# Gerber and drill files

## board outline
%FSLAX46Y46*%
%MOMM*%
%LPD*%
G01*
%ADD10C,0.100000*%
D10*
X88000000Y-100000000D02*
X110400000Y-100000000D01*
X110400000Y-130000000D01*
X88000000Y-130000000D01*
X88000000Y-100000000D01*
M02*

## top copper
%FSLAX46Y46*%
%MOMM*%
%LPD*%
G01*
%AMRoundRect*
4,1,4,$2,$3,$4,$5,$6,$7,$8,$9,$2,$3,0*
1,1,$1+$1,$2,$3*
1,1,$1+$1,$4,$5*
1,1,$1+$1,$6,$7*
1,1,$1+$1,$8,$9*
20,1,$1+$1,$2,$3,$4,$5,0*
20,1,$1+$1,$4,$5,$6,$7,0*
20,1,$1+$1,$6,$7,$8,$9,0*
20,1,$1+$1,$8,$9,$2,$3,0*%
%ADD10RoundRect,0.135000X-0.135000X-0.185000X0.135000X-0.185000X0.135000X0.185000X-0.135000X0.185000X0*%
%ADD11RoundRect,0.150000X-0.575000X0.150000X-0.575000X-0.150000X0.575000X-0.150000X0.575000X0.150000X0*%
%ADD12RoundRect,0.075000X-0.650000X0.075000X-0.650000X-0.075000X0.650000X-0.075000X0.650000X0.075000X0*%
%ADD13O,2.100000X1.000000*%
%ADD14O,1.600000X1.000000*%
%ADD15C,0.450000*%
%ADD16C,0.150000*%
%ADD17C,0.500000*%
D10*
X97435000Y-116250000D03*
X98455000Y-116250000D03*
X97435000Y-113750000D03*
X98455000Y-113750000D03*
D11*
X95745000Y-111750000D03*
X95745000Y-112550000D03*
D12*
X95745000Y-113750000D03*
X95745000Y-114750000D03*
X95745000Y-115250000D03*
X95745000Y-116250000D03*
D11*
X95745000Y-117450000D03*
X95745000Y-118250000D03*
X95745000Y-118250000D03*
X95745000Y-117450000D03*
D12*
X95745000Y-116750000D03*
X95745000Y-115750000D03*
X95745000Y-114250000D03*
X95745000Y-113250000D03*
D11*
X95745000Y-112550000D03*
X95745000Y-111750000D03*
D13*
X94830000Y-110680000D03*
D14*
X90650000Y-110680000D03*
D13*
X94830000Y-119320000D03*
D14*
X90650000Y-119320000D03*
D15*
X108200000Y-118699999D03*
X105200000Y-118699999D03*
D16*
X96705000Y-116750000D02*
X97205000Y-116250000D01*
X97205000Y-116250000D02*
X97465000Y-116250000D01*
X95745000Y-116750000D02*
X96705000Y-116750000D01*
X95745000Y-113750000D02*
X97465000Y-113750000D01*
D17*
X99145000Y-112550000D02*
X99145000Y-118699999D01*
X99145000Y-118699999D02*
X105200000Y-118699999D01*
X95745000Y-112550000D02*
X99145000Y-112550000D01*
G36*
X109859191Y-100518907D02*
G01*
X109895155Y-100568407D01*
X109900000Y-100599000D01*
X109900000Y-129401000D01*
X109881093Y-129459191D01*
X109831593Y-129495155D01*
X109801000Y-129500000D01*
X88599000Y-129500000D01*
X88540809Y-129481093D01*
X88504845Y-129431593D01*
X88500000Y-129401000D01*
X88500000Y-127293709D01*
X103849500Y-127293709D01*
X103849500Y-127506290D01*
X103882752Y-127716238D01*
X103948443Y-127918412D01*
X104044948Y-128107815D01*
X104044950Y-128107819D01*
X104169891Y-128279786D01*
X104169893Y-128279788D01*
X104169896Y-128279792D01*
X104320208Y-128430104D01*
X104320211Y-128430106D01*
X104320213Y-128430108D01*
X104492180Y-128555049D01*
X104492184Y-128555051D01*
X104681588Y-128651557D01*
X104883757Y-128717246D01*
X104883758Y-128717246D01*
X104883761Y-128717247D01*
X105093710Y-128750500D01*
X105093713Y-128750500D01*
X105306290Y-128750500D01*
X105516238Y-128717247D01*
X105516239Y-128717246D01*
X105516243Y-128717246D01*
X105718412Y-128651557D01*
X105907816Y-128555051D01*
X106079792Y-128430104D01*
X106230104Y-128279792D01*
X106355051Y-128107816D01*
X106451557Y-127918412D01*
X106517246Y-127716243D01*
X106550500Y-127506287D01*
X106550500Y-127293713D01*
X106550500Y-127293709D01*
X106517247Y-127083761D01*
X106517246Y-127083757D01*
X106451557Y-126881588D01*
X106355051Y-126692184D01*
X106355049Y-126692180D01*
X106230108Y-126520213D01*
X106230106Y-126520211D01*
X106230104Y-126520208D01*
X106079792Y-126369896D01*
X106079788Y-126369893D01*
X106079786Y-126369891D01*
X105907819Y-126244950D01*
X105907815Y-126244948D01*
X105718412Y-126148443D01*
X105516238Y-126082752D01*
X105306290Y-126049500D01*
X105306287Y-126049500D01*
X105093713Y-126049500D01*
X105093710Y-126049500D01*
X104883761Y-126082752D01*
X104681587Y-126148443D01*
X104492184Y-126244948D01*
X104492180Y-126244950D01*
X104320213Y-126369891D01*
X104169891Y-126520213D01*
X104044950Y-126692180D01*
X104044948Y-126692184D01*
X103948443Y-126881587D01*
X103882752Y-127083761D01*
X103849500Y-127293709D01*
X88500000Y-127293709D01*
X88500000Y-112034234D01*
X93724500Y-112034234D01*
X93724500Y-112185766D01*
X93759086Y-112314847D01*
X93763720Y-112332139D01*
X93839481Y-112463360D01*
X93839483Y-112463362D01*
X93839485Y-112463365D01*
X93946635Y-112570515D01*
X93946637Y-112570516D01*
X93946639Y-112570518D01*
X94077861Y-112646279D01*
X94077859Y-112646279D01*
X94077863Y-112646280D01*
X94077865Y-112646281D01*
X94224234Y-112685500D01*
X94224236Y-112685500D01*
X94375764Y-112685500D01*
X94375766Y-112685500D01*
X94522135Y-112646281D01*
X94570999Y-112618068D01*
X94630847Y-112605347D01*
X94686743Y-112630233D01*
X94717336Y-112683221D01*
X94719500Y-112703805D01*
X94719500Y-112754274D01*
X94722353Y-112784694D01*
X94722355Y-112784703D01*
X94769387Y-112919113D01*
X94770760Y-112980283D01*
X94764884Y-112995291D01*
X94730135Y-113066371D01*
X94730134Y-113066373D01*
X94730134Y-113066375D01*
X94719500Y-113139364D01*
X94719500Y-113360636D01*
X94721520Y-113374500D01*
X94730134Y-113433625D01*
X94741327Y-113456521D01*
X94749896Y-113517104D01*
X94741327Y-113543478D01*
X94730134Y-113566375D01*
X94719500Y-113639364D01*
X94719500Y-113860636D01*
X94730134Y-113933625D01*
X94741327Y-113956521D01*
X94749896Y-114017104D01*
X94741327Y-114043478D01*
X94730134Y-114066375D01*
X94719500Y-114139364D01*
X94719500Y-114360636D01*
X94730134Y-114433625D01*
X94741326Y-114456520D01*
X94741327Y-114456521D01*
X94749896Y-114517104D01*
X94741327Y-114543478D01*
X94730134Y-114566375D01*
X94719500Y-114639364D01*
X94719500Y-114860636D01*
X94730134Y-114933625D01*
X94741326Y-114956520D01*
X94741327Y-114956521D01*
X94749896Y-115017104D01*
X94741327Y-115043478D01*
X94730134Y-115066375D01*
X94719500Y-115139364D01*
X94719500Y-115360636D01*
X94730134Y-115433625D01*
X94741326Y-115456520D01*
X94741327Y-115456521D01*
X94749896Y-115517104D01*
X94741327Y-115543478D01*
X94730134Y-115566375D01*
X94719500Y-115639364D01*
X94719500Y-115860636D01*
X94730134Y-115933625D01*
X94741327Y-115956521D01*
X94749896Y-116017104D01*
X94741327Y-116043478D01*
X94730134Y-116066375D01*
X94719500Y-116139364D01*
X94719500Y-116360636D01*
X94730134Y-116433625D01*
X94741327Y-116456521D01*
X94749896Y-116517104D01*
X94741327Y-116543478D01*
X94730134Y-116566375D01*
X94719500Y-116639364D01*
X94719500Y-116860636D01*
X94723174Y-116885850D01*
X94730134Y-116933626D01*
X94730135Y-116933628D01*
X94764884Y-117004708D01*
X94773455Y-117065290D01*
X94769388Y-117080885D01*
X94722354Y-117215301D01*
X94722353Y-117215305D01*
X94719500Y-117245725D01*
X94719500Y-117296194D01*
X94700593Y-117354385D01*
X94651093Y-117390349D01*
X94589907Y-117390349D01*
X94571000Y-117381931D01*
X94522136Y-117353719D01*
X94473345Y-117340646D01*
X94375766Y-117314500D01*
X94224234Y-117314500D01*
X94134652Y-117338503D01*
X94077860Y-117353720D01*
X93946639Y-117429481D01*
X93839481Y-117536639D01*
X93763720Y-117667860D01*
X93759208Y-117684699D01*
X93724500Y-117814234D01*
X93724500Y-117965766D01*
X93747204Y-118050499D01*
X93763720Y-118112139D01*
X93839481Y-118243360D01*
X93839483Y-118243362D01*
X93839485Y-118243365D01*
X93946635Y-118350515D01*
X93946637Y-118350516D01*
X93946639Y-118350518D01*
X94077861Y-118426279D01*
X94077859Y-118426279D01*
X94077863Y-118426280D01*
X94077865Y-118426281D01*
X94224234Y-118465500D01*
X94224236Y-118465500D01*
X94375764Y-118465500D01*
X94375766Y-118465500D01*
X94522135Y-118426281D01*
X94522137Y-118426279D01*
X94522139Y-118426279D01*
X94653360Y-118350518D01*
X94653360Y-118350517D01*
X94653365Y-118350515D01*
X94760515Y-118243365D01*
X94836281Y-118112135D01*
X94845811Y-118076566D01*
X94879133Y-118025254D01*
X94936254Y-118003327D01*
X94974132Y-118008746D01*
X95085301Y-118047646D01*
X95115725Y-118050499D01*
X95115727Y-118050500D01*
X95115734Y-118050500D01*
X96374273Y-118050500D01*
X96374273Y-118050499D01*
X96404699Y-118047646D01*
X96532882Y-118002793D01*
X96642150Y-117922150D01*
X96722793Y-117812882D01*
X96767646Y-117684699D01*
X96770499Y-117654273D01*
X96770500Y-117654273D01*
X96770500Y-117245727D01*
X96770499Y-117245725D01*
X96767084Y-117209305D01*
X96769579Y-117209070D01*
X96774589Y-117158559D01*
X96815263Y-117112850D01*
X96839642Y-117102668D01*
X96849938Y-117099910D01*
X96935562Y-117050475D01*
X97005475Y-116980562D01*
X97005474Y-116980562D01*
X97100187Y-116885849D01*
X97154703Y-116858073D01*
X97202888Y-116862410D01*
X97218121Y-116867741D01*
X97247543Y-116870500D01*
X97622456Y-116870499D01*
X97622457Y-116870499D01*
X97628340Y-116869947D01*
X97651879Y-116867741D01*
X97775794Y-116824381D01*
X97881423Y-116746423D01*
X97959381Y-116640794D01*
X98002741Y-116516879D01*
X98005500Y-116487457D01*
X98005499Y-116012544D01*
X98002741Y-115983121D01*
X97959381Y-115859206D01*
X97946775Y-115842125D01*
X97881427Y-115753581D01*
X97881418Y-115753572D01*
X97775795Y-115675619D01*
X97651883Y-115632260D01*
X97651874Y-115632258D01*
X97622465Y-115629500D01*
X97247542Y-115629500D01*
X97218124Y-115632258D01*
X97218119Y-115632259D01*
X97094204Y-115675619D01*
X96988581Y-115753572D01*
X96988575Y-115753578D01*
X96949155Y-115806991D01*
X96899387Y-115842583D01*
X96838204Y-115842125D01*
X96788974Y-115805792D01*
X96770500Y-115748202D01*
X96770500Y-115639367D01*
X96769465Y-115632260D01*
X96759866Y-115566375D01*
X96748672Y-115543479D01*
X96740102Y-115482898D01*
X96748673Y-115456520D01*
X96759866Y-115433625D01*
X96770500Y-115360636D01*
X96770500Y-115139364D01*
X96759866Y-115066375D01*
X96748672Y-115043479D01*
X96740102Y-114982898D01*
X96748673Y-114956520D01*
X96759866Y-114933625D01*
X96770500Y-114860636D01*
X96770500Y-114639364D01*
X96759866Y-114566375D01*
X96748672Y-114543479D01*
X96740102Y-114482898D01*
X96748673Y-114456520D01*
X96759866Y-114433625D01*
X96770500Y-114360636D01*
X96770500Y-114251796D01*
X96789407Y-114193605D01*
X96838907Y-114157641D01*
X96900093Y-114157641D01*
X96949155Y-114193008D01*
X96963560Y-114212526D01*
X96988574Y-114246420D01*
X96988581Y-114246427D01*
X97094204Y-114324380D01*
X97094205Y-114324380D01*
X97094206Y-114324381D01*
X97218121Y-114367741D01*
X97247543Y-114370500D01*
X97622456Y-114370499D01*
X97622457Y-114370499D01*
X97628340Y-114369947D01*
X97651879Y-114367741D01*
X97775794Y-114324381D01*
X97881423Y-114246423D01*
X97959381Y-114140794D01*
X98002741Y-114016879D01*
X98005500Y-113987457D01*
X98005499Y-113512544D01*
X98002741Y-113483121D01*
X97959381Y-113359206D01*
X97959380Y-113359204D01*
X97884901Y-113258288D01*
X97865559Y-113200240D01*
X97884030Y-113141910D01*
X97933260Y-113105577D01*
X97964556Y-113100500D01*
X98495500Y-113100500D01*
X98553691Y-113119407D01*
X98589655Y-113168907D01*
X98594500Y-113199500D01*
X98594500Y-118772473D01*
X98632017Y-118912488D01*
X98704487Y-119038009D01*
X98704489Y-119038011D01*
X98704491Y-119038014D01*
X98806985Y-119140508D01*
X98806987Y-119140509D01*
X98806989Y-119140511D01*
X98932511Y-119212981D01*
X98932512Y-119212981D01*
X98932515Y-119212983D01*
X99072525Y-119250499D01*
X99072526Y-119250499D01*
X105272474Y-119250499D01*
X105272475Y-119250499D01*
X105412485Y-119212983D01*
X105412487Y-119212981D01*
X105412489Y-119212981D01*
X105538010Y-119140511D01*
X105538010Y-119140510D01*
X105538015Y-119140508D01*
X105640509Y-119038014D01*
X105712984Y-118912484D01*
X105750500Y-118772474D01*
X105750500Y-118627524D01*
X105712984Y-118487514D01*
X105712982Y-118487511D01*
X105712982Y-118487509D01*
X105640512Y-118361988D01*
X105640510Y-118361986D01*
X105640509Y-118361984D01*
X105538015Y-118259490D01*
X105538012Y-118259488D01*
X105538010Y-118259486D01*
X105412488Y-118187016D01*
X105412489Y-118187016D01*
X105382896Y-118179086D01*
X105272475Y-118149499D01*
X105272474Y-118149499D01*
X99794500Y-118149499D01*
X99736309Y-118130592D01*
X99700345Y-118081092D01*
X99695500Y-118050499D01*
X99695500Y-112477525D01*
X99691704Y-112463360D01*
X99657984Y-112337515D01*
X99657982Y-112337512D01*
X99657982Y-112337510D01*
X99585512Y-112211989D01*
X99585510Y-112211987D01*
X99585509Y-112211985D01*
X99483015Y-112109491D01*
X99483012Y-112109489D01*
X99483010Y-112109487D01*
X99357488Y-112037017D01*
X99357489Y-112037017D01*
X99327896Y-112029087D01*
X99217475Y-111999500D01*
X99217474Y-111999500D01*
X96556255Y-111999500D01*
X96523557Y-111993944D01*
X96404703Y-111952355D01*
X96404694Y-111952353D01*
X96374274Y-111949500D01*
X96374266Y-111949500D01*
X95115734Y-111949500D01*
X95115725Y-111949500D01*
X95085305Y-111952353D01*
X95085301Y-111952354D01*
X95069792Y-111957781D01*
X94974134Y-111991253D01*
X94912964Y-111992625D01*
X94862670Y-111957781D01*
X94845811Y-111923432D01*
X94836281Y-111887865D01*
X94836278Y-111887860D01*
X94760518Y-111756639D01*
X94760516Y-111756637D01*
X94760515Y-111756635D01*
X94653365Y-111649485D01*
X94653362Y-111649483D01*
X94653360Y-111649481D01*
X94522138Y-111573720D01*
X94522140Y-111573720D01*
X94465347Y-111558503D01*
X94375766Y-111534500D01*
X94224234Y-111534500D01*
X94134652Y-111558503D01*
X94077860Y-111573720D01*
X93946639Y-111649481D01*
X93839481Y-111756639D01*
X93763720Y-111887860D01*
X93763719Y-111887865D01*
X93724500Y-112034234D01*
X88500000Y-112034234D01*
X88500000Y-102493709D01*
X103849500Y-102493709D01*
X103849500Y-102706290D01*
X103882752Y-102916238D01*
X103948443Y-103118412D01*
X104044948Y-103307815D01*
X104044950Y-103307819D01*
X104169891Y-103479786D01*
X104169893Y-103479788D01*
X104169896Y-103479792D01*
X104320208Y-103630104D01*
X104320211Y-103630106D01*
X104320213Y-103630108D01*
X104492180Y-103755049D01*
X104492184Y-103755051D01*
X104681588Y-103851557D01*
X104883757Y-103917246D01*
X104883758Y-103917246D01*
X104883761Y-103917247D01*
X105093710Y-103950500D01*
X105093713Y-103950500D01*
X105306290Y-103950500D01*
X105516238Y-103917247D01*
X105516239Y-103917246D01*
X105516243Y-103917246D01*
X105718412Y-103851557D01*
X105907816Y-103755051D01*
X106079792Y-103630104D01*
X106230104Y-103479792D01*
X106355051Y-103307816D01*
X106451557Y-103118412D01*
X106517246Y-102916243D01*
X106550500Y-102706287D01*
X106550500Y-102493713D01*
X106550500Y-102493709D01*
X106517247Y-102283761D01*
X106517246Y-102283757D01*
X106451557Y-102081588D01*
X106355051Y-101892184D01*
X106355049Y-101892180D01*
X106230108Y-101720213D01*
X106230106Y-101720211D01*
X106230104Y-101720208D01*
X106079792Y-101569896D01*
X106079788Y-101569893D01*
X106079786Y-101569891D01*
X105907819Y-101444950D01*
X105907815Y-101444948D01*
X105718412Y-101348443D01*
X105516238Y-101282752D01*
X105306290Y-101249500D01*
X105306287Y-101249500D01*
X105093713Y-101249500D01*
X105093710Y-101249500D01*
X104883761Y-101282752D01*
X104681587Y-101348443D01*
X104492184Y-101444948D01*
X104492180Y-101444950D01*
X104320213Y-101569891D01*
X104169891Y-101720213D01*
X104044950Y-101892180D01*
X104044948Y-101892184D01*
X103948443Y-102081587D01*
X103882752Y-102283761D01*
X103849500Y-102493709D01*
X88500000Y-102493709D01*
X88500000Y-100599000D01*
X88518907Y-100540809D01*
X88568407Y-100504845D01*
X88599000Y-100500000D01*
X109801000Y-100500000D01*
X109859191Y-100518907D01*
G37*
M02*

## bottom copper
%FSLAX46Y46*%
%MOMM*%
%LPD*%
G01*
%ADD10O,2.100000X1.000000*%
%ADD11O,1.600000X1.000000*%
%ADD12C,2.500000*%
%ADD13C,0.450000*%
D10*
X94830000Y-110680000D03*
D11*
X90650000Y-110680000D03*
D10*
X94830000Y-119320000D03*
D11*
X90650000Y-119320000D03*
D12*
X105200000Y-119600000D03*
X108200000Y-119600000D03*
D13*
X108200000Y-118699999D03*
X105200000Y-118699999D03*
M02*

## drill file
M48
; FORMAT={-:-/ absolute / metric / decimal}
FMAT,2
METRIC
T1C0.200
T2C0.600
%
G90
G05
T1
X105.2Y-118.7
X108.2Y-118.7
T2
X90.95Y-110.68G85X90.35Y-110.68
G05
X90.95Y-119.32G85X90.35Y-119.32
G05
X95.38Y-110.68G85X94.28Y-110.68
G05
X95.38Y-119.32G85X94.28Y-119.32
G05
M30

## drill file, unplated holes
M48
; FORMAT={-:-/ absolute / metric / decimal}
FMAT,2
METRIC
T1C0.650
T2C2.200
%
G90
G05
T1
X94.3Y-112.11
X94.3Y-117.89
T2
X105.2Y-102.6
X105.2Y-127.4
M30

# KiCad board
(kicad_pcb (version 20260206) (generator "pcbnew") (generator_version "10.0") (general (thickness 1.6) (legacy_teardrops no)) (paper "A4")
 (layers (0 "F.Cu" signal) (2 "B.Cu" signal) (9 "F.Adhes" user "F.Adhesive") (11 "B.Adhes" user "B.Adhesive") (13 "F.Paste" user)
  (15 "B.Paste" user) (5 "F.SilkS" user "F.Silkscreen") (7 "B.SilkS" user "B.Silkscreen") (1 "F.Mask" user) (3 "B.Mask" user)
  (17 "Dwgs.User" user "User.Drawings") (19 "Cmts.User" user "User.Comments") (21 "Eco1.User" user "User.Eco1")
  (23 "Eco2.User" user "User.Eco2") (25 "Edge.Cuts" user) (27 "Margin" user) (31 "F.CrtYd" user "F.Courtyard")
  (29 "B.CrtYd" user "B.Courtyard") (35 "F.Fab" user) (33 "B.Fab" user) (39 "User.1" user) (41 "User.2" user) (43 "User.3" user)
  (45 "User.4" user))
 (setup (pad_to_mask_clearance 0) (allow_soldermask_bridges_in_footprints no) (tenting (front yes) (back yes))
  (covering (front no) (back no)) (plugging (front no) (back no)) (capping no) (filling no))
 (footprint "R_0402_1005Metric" (layer "F.Cu") (at 97.945 116.25)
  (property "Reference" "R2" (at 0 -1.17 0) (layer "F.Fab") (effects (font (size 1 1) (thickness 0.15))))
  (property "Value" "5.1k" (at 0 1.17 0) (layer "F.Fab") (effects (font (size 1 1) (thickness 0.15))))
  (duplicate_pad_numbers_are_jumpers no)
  (pad "1" smd roundrect (at -0.51 0) (size 0.54 0.64) (layers "F.Cu" "F.Mask" "F.Paste") (roundrect_rratio 0.25) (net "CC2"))
  (pad "2" smd roundrect (at 0.51 0) (size 0.54 0.64) (layers "F.Cu" "F.Mask" "F.Paste") (roundrect_rratio 0.25) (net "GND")))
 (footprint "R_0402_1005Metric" (layer "F.Cu") (at 97.945 113.75)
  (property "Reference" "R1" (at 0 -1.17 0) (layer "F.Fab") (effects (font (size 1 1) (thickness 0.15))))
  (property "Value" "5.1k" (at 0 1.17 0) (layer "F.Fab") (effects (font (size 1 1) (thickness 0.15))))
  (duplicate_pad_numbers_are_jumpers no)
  (pad "1" smd roundrect (at -0.51 0) (size 0.54 0.64) (layers "F.Cu" "F.Mask" "F.Paste") (roundrect_rratio 0.25) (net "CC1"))
  (pad "2" smd roundrect (at 0.51 0) (size 0.54 0.64) (layers "F.Cu" "F.Mask" "F.Paste") (roundrect_rratio 0.25) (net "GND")))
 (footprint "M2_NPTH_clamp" (layer "F.Cu") (at 105.2 127.4)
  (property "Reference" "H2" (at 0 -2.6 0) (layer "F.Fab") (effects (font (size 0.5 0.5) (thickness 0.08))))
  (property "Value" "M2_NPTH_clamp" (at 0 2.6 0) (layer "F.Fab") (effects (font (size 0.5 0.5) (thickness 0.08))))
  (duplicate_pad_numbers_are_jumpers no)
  (pad "" np_thru_hole circle (at 0 0) (size 2.2 2.2) (drill 2.2) (layers "*.Cu" "*.Mask")))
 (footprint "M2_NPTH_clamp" (layer "F.Cu") (at 105.2 102.6)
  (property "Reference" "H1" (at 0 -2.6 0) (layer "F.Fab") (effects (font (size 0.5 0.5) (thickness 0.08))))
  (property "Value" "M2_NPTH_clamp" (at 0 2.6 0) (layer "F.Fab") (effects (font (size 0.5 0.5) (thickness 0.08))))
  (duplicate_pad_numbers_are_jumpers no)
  (pad "" np_thru_hole circle (at 0 0) (size 2.2 2.2) (drill 2.2) (layers "*.Cu" "*.Mask")))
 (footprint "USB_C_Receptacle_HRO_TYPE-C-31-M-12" (layer "F.Cu") (at 91.7 115 -90)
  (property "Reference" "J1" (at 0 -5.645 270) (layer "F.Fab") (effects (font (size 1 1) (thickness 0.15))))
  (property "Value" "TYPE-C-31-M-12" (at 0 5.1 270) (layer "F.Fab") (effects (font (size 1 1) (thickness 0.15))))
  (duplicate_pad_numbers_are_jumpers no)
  (pad "" np_thru_hole circle (at -2.89 -2.6 270) (size 0.65 0.65) (drill 0.65) (layers "*.Cu" "*.Mask"))
  (pad "" np_thru_hole circle (at 2.89 -2.6 270) (size 0.65 0.65) (drill 0.65) (layers "*.Cu" "*.Mask"))
  (pad "A1" smd roundrect (at -3.25 -4.045 270) (size 0.6 1.45) (layers "F.Cu" "F.Mask" "F.Paste") (roundrect_rratio 0.25) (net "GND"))
  (pad "A4" smd roundrect (at -2.45 -4.045 270) (size 0.6 1.45) (layers "F.Cu" "F.Mask" "F.Paste") (roundrect_rratio 0.25) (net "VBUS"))
  (pad "A5" smd roundrect (at -1.25 -4.045 270) (size 0.3 1.45) (layers "F.Cu" "F.Mask" "F.Paste") (roundrect_rratio 0.25) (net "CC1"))
  (pad "A6" smd roundrect (at -0.25 -4.045 270) (size 0.3 1.45) (layers "F.Cu" "F.Mask" "F.Paste") (roundrect_rratio 0.25))
  (pad "A7" smd roundrect (at 0.25 -4.045 270) (size 0.3 1.45) (layers "F.Cu" "F.Mask" "F.Paste") (roundrect_rratio 0.25))
  (pad "A8" smd roundrect (at 1.25 -4.045 270) (size 0.3 1.45) (layers "F.Cu" "F.Mask" "F.Paste") (roundrect_rratio 0.25))
  (pad "A9" smd roundrect (at 2.45 -4.045 270) (size 0.6 1.45) (layers "F.Cu" "F.Mask" "F.Paste") (roundrect_rratio 0.25) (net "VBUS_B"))
  (pad "A12" smd roundrect (at 3.25 -4.045 270) (size 0.6 1.45) (layers "F.Cu" "F.Mask" "F.Paste") (roundrect_rratio 0.25) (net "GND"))
  (pad "B1" smd roundrect (at 3.25 -4.045 270) (size 0.6 1.45) (layers "F.Cu" "F.Mask" "F.Paste") (roundrect_rratio 0.25) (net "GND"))
  (pad "B4" smd roundrect (at 2.45 -4.045 270) (size 0.6 1.45) (layers "F.Cu" "F.Mask" "F.Paste") (roundrect_rratio 0.25) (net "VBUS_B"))
  (pad "B5" smd roundrect (at 1.75 -4.045 270) (size 0.3 1.45) (layers "F.Cu" "F.Mask" "F.Paste") (roundrect_rratio 0.25) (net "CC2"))
  (pad "B6" smd roundrect (at 0.75 -4.045 270) (size 0.3 1.45) (layers "F.Cu" "F.Mask" "F.Paste") (roundrect_rratio 0.25))
  (pad "B7" smd roundrect (at -0.75 -4.045 270) (size 0.3 1.45) (layers "F.Cu" "F.Mask" "F.Paste") (roundrect_rratio 0.25))
  (pad "B8" smd roundrect (at -1.75 -4.045 270) (size 0.3 1.45) (layers "F.Cu" "F.Mask" "F.Paste") (roundrect_rratio 0.25))
  (pad "B9" smd roundrect (at -2.45 -4.045 270) (size 0.6 1.45) (layers "F.Cu" "F.Mask" "F.Paste") (roundrect_rratio 0.25) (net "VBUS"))
  (pad "B12" smd roundrect (at -3.25 -4.045 270) (size 0.6 1.45) (layers "F.Cu" "F.Mask" "F.Paste") (roundrect_rratio 0.25) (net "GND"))
  (pad "SH" thru_hole oval (at -4.32 -3.13 270) (size 1 2.1) (drill oval 0.6 1.7) (layers "*.Cu" "*.Mask") (remove_unused_layers no)
   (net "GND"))
  (pad "SH" thru_hole oval (at -4.32 1.05 270) (size 1 1.6) (drill oval 0.6 1.2) (layers "*.Cu" "*.Mask") (remove_unused_layers no)
   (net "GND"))
  (pad "SH" thru_hole oval (at 4.32 -3.13 270) (size 1 2.1) (drill oval 0.6 1.7) (layers "*.Cu" "*.Mask") (remove_unused_layers no)
   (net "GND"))
  (pad "SH" thru_hole oval (at 4.32 1.05 270) (size 1 1.6) (drill oval 0.6 1.2) (layers "*.Cu" "*.Mask") (remove_unused_layers no)
   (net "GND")))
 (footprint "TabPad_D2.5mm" (layer "B.Cu") (at 105.2 119.6 180)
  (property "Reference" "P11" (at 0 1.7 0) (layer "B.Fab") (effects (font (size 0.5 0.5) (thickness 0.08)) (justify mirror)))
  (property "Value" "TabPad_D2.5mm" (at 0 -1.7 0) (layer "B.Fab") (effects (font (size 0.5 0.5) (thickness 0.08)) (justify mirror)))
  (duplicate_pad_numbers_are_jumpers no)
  (pad "1" smd circle (at 0 0 180) (size 2.5 2.5) (layers "B.Cu" "B.Mask") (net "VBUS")))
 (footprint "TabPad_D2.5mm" (layer "B.Cu") (at 108.2 119.6 180)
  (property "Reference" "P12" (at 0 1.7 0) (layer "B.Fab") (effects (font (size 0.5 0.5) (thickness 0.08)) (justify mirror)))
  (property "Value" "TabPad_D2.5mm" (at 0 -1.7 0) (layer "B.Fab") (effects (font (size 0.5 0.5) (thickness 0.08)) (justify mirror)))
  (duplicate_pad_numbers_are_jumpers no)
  (pad "1" smd circle (at 0 0 180) (size 2.5 2.5) (layers "B.Cu" "B.Mask") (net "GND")))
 (gr_rect (start 88 100) (end 110.4 130) (stroke (width 0.1) (type default)) (fill no) (layer "Edge.Cuts"))
 (segment (start 96.705 116.75) (end 97.205 116.25) (width 0.15) (layer "F.Cu") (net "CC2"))
 (segment (start 97.205 116.25) (end 97.465 116.25) (width 0.15) (layer "F.Cu") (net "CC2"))
 (segment (start 95.745 116.75) (end 96.705 116.75) (width 0.15) (layer "F.Cu") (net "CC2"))
 (via (at 108.2 118.699999) (size 0.45) (drill 0.2) (layers "F.Cu" "B.Cu") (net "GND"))
 (segment (start 95.745 113.75) (end 97.465 113.75) (width 0.15) (layer "F.Cu") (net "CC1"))
 (segment (start 99.145 112.55) (end 99.145 118.699999) (width 0.5) (layer "F.Cu") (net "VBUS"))
 (segment (start 99.145 118.699999) (end 105.2 118.699999) (width 0.5) (layer "F.Cu") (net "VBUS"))
 (segment (start 95.745 112.55) (end 99.145 112.55) (width 0.5) (layer "F.Cu") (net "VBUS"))
 (via (at 105.2 118.699999) (size 0.45) (drill 0.2) (layers "F.Cu" "B.Cu") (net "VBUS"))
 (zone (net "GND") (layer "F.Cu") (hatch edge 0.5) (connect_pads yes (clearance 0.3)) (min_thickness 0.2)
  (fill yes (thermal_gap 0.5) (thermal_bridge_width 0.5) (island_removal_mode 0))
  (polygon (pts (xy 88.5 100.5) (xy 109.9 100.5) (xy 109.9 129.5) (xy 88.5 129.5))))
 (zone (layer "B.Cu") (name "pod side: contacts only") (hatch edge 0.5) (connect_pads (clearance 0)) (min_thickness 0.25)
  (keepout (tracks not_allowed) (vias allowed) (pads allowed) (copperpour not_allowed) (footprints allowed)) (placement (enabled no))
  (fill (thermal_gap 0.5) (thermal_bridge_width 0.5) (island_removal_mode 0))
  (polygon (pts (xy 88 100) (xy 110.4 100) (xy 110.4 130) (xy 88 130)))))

